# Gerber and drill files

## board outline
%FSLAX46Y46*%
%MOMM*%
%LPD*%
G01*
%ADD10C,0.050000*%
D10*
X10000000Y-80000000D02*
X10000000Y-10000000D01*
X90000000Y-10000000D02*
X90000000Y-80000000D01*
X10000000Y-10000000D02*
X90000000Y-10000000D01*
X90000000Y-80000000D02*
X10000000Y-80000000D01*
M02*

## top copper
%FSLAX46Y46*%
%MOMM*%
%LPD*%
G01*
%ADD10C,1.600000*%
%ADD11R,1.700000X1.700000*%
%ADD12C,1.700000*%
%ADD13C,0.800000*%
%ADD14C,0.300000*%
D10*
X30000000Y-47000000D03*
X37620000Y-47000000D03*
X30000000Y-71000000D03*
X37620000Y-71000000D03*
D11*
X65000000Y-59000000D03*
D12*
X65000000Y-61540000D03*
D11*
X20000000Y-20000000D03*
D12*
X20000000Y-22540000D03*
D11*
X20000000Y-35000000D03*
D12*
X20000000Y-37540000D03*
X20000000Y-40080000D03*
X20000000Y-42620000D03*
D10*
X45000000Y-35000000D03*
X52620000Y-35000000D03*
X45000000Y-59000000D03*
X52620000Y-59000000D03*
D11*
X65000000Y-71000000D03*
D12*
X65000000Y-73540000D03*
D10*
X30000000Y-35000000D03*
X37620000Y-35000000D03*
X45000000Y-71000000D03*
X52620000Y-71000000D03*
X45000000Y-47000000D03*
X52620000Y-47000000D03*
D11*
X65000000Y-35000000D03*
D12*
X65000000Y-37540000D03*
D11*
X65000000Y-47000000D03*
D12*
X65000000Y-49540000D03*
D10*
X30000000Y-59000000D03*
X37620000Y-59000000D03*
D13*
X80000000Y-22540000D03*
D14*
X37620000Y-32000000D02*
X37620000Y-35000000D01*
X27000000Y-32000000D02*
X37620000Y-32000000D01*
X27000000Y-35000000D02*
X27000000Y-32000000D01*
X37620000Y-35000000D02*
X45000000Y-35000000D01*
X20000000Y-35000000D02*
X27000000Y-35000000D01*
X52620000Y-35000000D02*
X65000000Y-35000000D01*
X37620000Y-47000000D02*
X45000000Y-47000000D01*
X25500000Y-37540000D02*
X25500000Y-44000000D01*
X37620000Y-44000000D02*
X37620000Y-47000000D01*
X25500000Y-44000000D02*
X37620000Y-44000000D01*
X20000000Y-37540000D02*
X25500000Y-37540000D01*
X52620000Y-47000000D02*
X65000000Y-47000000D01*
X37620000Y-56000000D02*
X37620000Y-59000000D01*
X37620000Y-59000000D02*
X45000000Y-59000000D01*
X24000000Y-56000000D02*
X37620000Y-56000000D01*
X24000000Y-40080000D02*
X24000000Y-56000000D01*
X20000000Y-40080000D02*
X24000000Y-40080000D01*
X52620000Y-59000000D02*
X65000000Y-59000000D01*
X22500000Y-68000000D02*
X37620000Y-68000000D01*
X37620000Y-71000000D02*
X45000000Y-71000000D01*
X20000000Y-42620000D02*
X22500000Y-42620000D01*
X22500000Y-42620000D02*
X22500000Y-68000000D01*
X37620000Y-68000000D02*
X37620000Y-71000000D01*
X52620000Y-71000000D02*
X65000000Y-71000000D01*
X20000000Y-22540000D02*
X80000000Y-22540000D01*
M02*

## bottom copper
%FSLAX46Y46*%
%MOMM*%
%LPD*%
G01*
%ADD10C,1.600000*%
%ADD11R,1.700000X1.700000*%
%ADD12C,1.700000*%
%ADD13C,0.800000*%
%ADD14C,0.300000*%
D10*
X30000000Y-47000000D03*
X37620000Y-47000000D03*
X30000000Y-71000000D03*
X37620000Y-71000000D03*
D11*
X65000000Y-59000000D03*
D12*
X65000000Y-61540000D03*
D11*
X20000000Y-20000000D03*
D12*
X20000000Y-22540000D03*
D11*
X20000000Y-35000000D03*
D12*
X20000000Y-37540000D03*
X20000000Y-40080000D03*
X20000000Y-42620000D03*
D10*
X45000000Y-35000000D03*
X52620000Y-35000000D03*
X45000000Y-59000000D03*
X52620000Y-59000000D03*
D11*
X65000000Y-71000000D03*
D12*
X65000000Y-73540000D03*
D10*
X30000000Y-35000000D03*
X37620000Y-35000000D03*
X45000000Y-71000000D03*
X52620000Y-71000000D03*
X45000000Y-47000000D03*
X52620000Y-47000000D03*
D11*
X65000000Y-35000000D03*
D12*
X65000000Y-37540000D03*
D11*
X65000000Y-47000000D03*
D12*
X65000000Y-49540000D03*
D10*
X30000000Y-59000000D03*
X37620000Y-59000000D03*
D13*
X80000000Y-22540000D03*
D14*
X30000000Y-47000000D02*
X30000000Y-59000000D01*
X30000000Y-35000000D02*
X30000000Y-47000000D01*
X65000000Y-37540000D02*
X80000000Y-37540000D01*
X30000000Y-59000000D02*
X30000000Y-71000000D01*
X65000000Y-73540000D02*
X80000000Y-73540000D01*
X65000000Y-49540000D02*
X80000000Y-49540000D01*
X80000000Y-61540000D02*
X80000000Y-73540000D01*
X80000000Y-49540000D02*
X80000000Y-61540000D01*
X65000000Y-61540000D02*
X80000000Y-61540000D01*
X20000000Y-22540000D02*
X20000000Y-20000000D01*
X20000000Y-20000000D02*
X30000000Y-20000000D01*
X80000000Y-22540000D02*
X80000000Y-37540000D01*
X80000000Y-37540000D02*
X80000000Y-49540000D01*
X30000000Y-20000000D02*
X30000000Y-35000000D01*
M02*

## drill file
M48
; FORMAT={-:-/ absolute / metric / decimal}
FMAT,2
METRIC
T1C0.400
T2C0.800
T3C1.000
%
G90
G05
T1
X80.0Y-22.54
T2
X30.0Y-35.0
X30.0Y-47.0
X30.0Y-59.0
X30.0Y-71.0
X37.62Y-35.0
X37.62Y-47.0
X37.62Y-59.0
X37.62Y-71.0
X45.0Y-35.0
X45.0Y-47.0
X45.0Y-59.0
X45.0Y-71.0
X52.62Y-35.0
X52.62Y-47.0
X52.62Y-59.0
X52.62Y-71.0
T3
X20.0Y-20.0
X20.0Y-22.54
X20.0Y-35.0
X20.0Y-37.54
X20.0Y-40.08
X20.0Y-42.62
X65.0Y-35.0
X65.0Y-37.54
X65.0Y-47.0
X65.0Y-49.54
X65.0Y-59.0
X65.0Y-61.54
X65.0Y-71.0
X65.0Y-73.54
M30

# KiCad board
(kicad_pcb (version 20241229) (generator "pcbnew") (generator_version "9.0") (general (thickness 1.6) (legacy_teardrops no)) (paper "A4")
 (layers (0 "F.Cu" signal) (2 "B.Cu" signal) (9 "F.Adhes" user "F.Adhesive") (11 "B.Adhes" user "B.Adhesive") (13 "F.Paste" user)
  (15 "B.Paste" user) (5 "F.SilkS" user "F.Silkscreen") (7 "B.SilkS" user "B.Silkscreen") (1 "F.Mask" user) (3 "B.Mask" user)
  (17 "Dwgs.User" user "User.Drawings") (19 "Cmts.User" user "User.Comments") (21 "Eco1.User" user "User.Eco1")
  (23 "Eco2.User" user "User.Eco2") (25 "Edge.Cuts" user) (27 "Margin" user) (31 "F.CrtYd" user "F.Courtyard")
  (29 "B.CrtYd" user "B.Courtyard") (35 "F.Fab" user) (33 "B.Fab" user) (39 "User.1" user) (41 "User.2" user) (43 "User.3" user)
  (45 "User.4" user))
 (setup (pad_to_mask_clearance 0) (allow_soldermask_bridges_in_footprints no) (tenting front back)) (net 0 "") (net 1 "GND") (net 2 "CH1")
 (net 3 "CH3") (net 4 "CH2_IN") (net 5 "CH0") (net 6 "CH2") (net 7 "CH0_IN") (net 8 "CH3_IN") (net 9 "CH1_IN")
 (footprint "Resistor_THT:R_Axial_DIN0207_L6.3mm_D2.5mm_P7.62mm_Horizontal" (layer "F.Cu") (at 30 47)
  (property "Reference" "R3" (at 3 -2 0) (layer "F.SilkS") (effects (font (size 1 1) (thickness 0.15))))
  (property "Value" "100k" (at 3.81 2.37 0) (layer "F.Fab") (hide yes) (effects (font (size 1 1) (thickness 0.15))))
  (pad "1" thru_hole circle (at 0 0) (size 1.6 1.6) (drill 0.8) (layers "*.Cu" "*.Mask") (remove_unused_layers no) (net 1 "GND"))
  (pad "2" thru_hole circle (at 7.62 0) (size 1.6 1.6) (drill 0.8) (layers "*.Cu" "*.Mask") (remove_unused_layers no) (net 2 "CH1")))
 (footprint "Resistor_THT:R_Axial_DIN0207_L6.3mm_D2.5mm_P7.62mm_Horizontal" (layer "F.Cu") (at 30 71)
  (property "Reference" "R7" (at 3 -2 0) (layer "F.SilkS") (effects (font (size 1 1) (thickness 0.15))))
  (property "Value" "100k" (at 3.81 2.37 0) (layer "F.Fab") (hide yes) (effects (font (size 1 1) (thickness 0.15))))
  (pad "1" thru_hole circle (at 0 0) (size 1.6 1.6) (drill 0.8) (layers "*.Cu" "*.Mask") (remove_unused_layers no) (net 1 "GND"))
  (pad "2" thru_hole circle (at 7.62 0) (size 1.6 1.6) (drill 0.8) (layers "*.Cu" "*.Mask") (remove_unused_layers no) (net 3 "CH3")))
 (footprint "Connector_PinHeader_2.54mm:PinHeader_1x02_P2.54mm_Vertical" (layer "F.Cu") (at 65 59)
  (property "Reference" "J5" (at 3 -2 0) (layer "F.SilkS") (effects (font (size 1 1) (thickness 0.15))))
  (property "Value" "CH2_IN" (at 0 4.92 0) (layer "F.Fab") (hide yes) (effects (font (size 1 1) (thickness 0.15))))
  (pad "1" thru_hole rect (at 0 0) (size 1.7 1.7) (drill 1) (layers "*.Cu" "*.Mask") (remove_unused_layers no) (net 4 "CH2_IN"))
  (pad "2" thru_hole circle (at 0 2.54) (size 1.7 1.7) (drill 1) (layers "*.Cu" "*.Mask") (remove_unused_layers no) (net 1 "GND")))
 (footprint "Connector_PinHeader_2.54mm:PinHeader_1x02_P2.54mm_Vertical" (layer "F.Cu") (at 20 20)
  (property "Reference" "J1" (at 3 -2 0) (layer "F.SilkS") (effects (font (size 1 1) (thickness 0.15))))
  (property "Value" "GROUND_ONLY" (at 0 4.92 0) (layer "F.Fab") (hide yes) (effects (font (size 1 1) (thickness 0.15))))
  (pad "1" thru_hole rect (at 0 0) (size 1.7 1.7) (drill 1) (layers "*.Cu" "*.Mask") (remove_unused_layers no) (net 1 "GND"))
  (pad "2" thru_hole circle (at 0 2.54) (size 1.7 1.7) (drill 1) (layers "*.Cu" "*.Mask") (remove_unused_layers no) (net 1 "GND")))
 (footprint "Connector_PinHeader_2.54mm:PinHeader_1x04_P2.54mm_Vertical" (layer "F.Cu") (at 20 35)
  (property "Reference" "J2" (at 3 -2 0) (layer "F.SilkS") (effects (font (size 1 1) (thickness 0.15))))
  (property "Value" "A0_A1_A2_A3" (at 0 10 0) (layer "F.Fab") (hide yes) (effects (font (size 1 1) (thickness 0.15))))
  (pad "1" thru_hole rect (at 0 0) (size 1.7 1.7) (drill 1) (layers "*.Cu" "*.Mask") (remove_unused_layers no) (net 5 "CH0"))
  (pad "2" thru_hole circle (at 0 2.54) (size 1.7 1.7) (drill 1) (layers "*.Cu" "*.Mask") (remove_unused_layers no) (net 2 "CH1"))
  (pad "3" thru_hole circle (at 0 5.08) (size 1.7 1.7) (drill 1) (layers "*.Cu" "*.Mask") (remove_unused_layers no) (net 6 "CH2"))
  (pad "4" thru_hole circle (at 0 7.62) (size 1.7 1.7) (drill 1) (layers "*.Cu" "*.Mask") (remove_unused_layers no) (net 3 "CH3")))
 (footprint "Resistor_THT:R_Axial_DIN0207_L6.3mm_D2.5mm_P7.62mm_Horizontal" (layer "F.Cu") (at 45 35)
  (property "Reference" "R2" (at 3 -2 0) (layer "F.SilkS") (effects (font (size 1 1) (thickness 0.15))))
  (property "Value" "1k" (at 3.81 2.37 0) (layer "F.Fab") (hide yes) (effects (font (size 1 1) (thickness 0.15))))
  (pad "1" thru_hole circle (at 0 0) (size 1.6 1.6) (drill 0.8) (layers "*.Cu" "*.Mask") (remove_unused_layers no) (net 5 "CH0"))
  (pad "2" thru_hole circle (at 7.62 0) (size 1.6 1.6) (drill 0.8) (layers "*.Cu" "*.Mask") (remove_unused_layers no) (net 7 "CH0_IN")))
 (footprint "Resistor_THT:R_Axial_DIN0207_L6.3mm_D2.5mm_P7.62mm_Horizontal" (layer "F.Cu") (at 45 59)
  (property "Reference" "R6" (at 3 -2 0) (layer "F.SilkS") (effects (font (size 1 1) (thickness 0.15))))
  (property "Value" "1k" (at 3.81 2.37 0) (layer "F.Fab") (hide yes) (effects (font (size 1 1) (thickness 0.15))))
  (pad "1" thru_hole circle (at 0 0) (size 1.6 1.6) (drill 0.8) (layers "*.Cu" "*.Mask") (remove_unused_layers no) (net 6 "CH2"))
  (pad "2" thru_hole circle (at 7.62 0) (size 1.6 1.6) (drill 0.8) (layers "*.Cu" "*.Mask") (remove_unused_layers no) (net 4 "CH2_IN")))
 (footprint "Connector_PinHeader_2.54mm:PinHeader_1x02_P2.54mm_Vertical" (layer "F.Cu") (at 65 71)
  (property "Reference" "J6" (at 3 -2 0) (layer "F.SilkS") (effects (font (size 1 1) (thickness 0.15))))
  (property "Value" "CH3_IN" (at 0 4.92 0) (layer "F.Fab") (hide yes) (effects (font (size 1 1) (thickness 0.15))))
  (pad "1" thru_hole rect (at 0 0) (size 1.7 1.7) (drill 1) (layers "*.Cu" "*.Mask") (remove_unused_layers no) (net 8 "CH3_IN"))
  (pad "2" thru_hole circle (at 0 2.54) (size 1.7 1.7) (drill 1) (layers "*.Cu" "*.Mask") (remove_unused_layers no) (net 1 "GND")))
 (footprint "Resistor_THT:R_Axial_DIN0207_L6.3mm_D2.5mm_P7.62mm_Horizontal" (layer "F.Cu") (at 30 35)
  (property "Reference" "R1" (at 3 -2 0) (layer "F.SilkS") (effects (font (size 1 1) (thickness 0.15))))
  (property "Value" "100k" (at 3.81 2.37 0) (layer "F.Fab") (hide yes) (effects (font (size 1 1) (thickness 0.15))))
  (pad "1" thru_hole circle (at 0 0) (size 1.6 1.6) (drill 0.8) (layers "*.Cu" "*.Mask") (remove_unused_layers no) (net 1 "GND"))
  (pad "2" thru_hole circle (at 7.62 0) (size 1.6 1.6) (drill 0.8) (layers "*.Cu" "*.Mask") (remove_unused_layers no) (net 5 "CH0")))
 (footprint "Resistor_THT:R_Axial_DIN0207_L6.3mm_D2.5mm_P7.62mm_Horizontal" (layer "F.Cu") (at 45 71)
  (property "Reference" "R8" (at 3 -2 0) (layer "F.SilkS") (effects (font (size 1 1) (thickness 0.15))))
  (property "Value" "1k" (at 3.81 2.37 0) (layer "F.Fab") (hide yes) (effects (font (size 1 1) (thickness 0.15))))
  (pad "1" thru_hole circle (at 0 0) (size 1.6 1.6) (drill 0.8) (layers "*.Cu" "*.Mask") (remove_unused_layers no) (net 3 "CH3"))
  (pad "2" thru_hole circle (at 7.62 0) (size 1.6 1.6) (drill 0.8) (layers "*.Cu" "*.Mask") (remove_unused_layers no) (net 8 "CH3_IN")))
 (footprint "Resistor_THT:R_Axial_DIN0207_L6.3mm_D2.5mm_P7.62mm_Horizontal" (layer "F.Cu") (at 45 47)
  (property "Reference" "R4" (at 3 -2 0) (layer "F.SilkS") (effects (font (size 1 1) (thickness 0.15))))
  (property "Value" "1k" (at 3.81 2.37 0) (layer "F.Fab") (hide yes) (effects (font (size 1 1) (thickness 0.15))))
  (pad "1" thru_hole circle (at 0 0) (size 1.6 1.6) (drill 0.8) (layers "*.Cu" "*.Mask") (remove_unused_layers no) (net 2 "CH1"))
  (pad "2" thru_hole circle (at 7.62 0) (size 1.6 1.6) (drill 0.8) (layers "*.Cu" "*.Mask") (remove_unused_layers no) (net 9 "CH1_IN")))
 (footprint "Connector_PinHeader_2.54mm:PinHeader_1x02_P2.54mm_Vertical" (layer "F.Cu") (at 65 35)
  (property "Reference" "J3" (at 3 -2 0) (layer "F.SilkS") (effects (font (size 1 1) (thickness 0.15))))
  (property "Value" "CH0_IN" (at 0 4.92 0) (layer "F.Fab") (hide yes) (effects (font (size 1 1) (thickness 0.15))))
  (pad "1" thru_hole rect (at 0 0) (size 1.7 1.7) (drill 1) (layers "*.Cu" "*.Mask") (remove_unused_layers no) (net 7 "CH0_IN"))
  (pad "2" thru_hole circle (at 0 2.54) (size 1.7 1.7) (drill 1) (layers "*.Cu" "*.Mask") (remove_unused_layers no) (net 1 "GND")))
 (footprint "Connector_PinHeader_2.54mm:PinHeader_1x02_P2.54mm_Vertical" (layer "F.Cu") (at 65 47)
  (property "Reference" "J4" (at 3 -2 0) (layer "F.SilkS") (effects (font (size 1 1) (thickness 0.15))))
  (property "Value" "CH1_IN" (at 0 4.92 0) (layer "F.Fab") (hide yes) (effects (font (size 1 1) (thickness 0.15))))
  (pad "1" thru_hole rect (at 0 0) (size 1.7 1.7) (drill 1) (layers "*.Cu" "*.Mask") (remove_unused_layers no) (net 9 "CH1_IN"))
  (pad "2" thru_hole circle (at 0 2.54) (size 1.7 1.7) (drill 1) (layers "*.Cu" "*.Mask") (remove_unused_layers no) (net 1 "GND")))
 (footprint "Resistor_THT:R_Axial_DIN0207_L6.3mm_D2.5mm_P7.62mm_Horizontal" (layer "F.Cu") (at 30 59)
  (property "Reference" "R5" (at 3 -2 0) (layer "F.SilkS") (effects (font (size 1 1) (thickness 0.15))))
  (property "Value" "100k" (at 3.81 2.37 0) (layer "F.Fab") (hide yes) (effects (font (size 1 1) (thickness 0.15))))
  (pad "1" thru_hole circle (at 0 0) (size 1.6 1.6) (drill 0.8) (layers "*.Cu" "*.Mask") (remove_unused_layers no) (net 1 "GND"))
  (pad "2" thru_hole circle (at 7.62 0) (size 1.6 1.6) (drill 0.8) (layers "*.Cu" "*.Mask") (remove_unused_layers no) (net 6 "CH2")))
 (gr_line (start 10 80) (end 10 10) (stroke (width 0.05) (type default)) (layer "Edge.Cuts"))
 (gr_line (start 90 10) (end 90 80) (stroke (width 0.05) (type default)) (layer "Edge.Cuts"))
 (gr_line (start 10 10) (end 90 10) (stroke (width 0.05) (type default)) (layer "Edge.Cuts"))
 (gr_line (start 90 80) (end 10 80) (stroke (width 0.05) (type default)) (layer "Edge.Cuts"))
 (segment (start 37.62 32) (end 37.62 35) (width 0.3) (layer "F.Cu") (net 5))
 (segment (start 27 32) (end 37.62 32) (width 0.3) (layer "F.Cu") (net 5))
 (segment (start 27 35) (end 27 32) (width 0.3) (layer "F.Cu") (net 5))
 (segment (start 37.62 35) (end 45 35) (width 0.3) (layer "F.Cu") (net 5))
 (segment (start 20 35) (end 27 35) (width 0.3) (layer "F.Cu") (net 5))
 (segment (start 52.62 35) (end 65 35) (width 0.3) (layer "F.Cu") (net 7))
 (segment (start 37.62 47) (end 45 47) (width 0.3) (layer "F.Cu") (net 2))
 (segment (start 25.5 37.54) (end 25.5 44) (width 0.3) (layer "F.Cu") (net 2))
 (segment (start 37.62 44) (end 37.62 47) (width 0.3) (layer "F.Cu") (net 2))
 (segment (start 25.5 44) (end 37.62 44) (width 0.3) (layer "F.Cu") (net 2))
 (segment (start 20 37.54) (end 25.5 37.54) (width 0.3) (layer "F.Cu") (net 2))
 (segment (start 52.62 47) (end 65 47) (width 0.3) (layer "F.Cu") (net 9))
 (segment (start 37.62 56) (end 37.62 59) (width 0.3) (layer "F.Cu") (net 6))
 (segment (start 37.62 59) (end 45 59) (width 0.3) (layer "F.Cu") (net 6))
 (segment (start 24 56) (end 37.62 56) (width 0.3) (layer "F.Cu") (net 6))
 (segment (start 24 40.08) (end 24 56) (width 0.3) (layer "F.Cu") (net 6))
 (segment (start 20 40.08) (end 24 40.08) (width 0.3) (layer "F.Cu") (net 6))
 (segment (start 52.62 59) (end 65 59) (width 0.3) (layer "F.Cu") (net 4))
 (segment (start 22.5 68) (end 37.62 68) (width 0.3) (layer "F.Cu") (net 3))
 (segment (start 37.62 71) (end 45 71) (width 0.3) (layer "F.Cu") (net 3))
 (segment (start 20 42.62) (end 22.5 42.62) (width 0.3) (layer "F.Cu") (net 3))
 (segment (start 22.5 42.62) (end 22.5 68) (width 0.3) (layer "F.Cu") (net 3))
 (segment (start 37.62 68) (end 37.62 71) (width 0.3) (layer "F.Cu") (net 3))
 (segment (start 52.62 71) (end 65 71) (width 0.3) (layer "F.Cu") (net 8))
 (segment (start 20 22.54) (end 80 22.54) (width 0.3) (layer "F.Cu") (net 1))
 (via (at 80 22.54) (size 0.8) (drill 0.4) (layers "F.Cu" "B.Cu") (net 1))
 (segment (start 30 47) (end 30 59) (width 0.3) (layer "B.Cu") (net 1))
 (segment (start 30 35) (end 30 47) (width 0.3) (layer "B.Cu") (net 1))
 (segment (start 65 37.54) (end 80 37.54) (width 0.3) (layer "B.Cu") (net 1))
 (segment (start 30 59) (end 30 71) (width 0.3) (layer "B.Cu") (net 1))
 (segment (start 65 73.54) (end 80 73.54) (width 0.3) (layer "B.Cu") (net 1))
 (segment (start 65 49.54) (end 80 49.54) (width 0.3) (layer "B.Cu") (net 1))
 (segment (start 80 61.54) (end 80 73.54) (width 0.3) (layer "B.Cu") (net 1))
 (segment (start 80 49.54) (end 80 61.54) (width 0.3) (layer "B.Cu") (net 1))
 (segment (start 65 61.54) (end 80 61.54) (width 0.3) (layer "B.Cu") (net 1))
 (segment (start 20 22.54) (end 20 20) (width 0.3) (layer "B.Cu") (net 1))
 (segment (start 20 20) (end 30 20) (width 0.3) (layer "B.Cu") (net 1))
 (segment (start 80 22.54) (end 80 37.54) (width 0.3) (layer "B.Cu") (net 1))
 (segment (start 80 37.54) (end 80 49.54) (width 0.3) (layer "B.Cu") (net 1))
 (segment (start 30 20) (end 30 35) (width 0.3) (layer "B.Cu") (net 1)))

